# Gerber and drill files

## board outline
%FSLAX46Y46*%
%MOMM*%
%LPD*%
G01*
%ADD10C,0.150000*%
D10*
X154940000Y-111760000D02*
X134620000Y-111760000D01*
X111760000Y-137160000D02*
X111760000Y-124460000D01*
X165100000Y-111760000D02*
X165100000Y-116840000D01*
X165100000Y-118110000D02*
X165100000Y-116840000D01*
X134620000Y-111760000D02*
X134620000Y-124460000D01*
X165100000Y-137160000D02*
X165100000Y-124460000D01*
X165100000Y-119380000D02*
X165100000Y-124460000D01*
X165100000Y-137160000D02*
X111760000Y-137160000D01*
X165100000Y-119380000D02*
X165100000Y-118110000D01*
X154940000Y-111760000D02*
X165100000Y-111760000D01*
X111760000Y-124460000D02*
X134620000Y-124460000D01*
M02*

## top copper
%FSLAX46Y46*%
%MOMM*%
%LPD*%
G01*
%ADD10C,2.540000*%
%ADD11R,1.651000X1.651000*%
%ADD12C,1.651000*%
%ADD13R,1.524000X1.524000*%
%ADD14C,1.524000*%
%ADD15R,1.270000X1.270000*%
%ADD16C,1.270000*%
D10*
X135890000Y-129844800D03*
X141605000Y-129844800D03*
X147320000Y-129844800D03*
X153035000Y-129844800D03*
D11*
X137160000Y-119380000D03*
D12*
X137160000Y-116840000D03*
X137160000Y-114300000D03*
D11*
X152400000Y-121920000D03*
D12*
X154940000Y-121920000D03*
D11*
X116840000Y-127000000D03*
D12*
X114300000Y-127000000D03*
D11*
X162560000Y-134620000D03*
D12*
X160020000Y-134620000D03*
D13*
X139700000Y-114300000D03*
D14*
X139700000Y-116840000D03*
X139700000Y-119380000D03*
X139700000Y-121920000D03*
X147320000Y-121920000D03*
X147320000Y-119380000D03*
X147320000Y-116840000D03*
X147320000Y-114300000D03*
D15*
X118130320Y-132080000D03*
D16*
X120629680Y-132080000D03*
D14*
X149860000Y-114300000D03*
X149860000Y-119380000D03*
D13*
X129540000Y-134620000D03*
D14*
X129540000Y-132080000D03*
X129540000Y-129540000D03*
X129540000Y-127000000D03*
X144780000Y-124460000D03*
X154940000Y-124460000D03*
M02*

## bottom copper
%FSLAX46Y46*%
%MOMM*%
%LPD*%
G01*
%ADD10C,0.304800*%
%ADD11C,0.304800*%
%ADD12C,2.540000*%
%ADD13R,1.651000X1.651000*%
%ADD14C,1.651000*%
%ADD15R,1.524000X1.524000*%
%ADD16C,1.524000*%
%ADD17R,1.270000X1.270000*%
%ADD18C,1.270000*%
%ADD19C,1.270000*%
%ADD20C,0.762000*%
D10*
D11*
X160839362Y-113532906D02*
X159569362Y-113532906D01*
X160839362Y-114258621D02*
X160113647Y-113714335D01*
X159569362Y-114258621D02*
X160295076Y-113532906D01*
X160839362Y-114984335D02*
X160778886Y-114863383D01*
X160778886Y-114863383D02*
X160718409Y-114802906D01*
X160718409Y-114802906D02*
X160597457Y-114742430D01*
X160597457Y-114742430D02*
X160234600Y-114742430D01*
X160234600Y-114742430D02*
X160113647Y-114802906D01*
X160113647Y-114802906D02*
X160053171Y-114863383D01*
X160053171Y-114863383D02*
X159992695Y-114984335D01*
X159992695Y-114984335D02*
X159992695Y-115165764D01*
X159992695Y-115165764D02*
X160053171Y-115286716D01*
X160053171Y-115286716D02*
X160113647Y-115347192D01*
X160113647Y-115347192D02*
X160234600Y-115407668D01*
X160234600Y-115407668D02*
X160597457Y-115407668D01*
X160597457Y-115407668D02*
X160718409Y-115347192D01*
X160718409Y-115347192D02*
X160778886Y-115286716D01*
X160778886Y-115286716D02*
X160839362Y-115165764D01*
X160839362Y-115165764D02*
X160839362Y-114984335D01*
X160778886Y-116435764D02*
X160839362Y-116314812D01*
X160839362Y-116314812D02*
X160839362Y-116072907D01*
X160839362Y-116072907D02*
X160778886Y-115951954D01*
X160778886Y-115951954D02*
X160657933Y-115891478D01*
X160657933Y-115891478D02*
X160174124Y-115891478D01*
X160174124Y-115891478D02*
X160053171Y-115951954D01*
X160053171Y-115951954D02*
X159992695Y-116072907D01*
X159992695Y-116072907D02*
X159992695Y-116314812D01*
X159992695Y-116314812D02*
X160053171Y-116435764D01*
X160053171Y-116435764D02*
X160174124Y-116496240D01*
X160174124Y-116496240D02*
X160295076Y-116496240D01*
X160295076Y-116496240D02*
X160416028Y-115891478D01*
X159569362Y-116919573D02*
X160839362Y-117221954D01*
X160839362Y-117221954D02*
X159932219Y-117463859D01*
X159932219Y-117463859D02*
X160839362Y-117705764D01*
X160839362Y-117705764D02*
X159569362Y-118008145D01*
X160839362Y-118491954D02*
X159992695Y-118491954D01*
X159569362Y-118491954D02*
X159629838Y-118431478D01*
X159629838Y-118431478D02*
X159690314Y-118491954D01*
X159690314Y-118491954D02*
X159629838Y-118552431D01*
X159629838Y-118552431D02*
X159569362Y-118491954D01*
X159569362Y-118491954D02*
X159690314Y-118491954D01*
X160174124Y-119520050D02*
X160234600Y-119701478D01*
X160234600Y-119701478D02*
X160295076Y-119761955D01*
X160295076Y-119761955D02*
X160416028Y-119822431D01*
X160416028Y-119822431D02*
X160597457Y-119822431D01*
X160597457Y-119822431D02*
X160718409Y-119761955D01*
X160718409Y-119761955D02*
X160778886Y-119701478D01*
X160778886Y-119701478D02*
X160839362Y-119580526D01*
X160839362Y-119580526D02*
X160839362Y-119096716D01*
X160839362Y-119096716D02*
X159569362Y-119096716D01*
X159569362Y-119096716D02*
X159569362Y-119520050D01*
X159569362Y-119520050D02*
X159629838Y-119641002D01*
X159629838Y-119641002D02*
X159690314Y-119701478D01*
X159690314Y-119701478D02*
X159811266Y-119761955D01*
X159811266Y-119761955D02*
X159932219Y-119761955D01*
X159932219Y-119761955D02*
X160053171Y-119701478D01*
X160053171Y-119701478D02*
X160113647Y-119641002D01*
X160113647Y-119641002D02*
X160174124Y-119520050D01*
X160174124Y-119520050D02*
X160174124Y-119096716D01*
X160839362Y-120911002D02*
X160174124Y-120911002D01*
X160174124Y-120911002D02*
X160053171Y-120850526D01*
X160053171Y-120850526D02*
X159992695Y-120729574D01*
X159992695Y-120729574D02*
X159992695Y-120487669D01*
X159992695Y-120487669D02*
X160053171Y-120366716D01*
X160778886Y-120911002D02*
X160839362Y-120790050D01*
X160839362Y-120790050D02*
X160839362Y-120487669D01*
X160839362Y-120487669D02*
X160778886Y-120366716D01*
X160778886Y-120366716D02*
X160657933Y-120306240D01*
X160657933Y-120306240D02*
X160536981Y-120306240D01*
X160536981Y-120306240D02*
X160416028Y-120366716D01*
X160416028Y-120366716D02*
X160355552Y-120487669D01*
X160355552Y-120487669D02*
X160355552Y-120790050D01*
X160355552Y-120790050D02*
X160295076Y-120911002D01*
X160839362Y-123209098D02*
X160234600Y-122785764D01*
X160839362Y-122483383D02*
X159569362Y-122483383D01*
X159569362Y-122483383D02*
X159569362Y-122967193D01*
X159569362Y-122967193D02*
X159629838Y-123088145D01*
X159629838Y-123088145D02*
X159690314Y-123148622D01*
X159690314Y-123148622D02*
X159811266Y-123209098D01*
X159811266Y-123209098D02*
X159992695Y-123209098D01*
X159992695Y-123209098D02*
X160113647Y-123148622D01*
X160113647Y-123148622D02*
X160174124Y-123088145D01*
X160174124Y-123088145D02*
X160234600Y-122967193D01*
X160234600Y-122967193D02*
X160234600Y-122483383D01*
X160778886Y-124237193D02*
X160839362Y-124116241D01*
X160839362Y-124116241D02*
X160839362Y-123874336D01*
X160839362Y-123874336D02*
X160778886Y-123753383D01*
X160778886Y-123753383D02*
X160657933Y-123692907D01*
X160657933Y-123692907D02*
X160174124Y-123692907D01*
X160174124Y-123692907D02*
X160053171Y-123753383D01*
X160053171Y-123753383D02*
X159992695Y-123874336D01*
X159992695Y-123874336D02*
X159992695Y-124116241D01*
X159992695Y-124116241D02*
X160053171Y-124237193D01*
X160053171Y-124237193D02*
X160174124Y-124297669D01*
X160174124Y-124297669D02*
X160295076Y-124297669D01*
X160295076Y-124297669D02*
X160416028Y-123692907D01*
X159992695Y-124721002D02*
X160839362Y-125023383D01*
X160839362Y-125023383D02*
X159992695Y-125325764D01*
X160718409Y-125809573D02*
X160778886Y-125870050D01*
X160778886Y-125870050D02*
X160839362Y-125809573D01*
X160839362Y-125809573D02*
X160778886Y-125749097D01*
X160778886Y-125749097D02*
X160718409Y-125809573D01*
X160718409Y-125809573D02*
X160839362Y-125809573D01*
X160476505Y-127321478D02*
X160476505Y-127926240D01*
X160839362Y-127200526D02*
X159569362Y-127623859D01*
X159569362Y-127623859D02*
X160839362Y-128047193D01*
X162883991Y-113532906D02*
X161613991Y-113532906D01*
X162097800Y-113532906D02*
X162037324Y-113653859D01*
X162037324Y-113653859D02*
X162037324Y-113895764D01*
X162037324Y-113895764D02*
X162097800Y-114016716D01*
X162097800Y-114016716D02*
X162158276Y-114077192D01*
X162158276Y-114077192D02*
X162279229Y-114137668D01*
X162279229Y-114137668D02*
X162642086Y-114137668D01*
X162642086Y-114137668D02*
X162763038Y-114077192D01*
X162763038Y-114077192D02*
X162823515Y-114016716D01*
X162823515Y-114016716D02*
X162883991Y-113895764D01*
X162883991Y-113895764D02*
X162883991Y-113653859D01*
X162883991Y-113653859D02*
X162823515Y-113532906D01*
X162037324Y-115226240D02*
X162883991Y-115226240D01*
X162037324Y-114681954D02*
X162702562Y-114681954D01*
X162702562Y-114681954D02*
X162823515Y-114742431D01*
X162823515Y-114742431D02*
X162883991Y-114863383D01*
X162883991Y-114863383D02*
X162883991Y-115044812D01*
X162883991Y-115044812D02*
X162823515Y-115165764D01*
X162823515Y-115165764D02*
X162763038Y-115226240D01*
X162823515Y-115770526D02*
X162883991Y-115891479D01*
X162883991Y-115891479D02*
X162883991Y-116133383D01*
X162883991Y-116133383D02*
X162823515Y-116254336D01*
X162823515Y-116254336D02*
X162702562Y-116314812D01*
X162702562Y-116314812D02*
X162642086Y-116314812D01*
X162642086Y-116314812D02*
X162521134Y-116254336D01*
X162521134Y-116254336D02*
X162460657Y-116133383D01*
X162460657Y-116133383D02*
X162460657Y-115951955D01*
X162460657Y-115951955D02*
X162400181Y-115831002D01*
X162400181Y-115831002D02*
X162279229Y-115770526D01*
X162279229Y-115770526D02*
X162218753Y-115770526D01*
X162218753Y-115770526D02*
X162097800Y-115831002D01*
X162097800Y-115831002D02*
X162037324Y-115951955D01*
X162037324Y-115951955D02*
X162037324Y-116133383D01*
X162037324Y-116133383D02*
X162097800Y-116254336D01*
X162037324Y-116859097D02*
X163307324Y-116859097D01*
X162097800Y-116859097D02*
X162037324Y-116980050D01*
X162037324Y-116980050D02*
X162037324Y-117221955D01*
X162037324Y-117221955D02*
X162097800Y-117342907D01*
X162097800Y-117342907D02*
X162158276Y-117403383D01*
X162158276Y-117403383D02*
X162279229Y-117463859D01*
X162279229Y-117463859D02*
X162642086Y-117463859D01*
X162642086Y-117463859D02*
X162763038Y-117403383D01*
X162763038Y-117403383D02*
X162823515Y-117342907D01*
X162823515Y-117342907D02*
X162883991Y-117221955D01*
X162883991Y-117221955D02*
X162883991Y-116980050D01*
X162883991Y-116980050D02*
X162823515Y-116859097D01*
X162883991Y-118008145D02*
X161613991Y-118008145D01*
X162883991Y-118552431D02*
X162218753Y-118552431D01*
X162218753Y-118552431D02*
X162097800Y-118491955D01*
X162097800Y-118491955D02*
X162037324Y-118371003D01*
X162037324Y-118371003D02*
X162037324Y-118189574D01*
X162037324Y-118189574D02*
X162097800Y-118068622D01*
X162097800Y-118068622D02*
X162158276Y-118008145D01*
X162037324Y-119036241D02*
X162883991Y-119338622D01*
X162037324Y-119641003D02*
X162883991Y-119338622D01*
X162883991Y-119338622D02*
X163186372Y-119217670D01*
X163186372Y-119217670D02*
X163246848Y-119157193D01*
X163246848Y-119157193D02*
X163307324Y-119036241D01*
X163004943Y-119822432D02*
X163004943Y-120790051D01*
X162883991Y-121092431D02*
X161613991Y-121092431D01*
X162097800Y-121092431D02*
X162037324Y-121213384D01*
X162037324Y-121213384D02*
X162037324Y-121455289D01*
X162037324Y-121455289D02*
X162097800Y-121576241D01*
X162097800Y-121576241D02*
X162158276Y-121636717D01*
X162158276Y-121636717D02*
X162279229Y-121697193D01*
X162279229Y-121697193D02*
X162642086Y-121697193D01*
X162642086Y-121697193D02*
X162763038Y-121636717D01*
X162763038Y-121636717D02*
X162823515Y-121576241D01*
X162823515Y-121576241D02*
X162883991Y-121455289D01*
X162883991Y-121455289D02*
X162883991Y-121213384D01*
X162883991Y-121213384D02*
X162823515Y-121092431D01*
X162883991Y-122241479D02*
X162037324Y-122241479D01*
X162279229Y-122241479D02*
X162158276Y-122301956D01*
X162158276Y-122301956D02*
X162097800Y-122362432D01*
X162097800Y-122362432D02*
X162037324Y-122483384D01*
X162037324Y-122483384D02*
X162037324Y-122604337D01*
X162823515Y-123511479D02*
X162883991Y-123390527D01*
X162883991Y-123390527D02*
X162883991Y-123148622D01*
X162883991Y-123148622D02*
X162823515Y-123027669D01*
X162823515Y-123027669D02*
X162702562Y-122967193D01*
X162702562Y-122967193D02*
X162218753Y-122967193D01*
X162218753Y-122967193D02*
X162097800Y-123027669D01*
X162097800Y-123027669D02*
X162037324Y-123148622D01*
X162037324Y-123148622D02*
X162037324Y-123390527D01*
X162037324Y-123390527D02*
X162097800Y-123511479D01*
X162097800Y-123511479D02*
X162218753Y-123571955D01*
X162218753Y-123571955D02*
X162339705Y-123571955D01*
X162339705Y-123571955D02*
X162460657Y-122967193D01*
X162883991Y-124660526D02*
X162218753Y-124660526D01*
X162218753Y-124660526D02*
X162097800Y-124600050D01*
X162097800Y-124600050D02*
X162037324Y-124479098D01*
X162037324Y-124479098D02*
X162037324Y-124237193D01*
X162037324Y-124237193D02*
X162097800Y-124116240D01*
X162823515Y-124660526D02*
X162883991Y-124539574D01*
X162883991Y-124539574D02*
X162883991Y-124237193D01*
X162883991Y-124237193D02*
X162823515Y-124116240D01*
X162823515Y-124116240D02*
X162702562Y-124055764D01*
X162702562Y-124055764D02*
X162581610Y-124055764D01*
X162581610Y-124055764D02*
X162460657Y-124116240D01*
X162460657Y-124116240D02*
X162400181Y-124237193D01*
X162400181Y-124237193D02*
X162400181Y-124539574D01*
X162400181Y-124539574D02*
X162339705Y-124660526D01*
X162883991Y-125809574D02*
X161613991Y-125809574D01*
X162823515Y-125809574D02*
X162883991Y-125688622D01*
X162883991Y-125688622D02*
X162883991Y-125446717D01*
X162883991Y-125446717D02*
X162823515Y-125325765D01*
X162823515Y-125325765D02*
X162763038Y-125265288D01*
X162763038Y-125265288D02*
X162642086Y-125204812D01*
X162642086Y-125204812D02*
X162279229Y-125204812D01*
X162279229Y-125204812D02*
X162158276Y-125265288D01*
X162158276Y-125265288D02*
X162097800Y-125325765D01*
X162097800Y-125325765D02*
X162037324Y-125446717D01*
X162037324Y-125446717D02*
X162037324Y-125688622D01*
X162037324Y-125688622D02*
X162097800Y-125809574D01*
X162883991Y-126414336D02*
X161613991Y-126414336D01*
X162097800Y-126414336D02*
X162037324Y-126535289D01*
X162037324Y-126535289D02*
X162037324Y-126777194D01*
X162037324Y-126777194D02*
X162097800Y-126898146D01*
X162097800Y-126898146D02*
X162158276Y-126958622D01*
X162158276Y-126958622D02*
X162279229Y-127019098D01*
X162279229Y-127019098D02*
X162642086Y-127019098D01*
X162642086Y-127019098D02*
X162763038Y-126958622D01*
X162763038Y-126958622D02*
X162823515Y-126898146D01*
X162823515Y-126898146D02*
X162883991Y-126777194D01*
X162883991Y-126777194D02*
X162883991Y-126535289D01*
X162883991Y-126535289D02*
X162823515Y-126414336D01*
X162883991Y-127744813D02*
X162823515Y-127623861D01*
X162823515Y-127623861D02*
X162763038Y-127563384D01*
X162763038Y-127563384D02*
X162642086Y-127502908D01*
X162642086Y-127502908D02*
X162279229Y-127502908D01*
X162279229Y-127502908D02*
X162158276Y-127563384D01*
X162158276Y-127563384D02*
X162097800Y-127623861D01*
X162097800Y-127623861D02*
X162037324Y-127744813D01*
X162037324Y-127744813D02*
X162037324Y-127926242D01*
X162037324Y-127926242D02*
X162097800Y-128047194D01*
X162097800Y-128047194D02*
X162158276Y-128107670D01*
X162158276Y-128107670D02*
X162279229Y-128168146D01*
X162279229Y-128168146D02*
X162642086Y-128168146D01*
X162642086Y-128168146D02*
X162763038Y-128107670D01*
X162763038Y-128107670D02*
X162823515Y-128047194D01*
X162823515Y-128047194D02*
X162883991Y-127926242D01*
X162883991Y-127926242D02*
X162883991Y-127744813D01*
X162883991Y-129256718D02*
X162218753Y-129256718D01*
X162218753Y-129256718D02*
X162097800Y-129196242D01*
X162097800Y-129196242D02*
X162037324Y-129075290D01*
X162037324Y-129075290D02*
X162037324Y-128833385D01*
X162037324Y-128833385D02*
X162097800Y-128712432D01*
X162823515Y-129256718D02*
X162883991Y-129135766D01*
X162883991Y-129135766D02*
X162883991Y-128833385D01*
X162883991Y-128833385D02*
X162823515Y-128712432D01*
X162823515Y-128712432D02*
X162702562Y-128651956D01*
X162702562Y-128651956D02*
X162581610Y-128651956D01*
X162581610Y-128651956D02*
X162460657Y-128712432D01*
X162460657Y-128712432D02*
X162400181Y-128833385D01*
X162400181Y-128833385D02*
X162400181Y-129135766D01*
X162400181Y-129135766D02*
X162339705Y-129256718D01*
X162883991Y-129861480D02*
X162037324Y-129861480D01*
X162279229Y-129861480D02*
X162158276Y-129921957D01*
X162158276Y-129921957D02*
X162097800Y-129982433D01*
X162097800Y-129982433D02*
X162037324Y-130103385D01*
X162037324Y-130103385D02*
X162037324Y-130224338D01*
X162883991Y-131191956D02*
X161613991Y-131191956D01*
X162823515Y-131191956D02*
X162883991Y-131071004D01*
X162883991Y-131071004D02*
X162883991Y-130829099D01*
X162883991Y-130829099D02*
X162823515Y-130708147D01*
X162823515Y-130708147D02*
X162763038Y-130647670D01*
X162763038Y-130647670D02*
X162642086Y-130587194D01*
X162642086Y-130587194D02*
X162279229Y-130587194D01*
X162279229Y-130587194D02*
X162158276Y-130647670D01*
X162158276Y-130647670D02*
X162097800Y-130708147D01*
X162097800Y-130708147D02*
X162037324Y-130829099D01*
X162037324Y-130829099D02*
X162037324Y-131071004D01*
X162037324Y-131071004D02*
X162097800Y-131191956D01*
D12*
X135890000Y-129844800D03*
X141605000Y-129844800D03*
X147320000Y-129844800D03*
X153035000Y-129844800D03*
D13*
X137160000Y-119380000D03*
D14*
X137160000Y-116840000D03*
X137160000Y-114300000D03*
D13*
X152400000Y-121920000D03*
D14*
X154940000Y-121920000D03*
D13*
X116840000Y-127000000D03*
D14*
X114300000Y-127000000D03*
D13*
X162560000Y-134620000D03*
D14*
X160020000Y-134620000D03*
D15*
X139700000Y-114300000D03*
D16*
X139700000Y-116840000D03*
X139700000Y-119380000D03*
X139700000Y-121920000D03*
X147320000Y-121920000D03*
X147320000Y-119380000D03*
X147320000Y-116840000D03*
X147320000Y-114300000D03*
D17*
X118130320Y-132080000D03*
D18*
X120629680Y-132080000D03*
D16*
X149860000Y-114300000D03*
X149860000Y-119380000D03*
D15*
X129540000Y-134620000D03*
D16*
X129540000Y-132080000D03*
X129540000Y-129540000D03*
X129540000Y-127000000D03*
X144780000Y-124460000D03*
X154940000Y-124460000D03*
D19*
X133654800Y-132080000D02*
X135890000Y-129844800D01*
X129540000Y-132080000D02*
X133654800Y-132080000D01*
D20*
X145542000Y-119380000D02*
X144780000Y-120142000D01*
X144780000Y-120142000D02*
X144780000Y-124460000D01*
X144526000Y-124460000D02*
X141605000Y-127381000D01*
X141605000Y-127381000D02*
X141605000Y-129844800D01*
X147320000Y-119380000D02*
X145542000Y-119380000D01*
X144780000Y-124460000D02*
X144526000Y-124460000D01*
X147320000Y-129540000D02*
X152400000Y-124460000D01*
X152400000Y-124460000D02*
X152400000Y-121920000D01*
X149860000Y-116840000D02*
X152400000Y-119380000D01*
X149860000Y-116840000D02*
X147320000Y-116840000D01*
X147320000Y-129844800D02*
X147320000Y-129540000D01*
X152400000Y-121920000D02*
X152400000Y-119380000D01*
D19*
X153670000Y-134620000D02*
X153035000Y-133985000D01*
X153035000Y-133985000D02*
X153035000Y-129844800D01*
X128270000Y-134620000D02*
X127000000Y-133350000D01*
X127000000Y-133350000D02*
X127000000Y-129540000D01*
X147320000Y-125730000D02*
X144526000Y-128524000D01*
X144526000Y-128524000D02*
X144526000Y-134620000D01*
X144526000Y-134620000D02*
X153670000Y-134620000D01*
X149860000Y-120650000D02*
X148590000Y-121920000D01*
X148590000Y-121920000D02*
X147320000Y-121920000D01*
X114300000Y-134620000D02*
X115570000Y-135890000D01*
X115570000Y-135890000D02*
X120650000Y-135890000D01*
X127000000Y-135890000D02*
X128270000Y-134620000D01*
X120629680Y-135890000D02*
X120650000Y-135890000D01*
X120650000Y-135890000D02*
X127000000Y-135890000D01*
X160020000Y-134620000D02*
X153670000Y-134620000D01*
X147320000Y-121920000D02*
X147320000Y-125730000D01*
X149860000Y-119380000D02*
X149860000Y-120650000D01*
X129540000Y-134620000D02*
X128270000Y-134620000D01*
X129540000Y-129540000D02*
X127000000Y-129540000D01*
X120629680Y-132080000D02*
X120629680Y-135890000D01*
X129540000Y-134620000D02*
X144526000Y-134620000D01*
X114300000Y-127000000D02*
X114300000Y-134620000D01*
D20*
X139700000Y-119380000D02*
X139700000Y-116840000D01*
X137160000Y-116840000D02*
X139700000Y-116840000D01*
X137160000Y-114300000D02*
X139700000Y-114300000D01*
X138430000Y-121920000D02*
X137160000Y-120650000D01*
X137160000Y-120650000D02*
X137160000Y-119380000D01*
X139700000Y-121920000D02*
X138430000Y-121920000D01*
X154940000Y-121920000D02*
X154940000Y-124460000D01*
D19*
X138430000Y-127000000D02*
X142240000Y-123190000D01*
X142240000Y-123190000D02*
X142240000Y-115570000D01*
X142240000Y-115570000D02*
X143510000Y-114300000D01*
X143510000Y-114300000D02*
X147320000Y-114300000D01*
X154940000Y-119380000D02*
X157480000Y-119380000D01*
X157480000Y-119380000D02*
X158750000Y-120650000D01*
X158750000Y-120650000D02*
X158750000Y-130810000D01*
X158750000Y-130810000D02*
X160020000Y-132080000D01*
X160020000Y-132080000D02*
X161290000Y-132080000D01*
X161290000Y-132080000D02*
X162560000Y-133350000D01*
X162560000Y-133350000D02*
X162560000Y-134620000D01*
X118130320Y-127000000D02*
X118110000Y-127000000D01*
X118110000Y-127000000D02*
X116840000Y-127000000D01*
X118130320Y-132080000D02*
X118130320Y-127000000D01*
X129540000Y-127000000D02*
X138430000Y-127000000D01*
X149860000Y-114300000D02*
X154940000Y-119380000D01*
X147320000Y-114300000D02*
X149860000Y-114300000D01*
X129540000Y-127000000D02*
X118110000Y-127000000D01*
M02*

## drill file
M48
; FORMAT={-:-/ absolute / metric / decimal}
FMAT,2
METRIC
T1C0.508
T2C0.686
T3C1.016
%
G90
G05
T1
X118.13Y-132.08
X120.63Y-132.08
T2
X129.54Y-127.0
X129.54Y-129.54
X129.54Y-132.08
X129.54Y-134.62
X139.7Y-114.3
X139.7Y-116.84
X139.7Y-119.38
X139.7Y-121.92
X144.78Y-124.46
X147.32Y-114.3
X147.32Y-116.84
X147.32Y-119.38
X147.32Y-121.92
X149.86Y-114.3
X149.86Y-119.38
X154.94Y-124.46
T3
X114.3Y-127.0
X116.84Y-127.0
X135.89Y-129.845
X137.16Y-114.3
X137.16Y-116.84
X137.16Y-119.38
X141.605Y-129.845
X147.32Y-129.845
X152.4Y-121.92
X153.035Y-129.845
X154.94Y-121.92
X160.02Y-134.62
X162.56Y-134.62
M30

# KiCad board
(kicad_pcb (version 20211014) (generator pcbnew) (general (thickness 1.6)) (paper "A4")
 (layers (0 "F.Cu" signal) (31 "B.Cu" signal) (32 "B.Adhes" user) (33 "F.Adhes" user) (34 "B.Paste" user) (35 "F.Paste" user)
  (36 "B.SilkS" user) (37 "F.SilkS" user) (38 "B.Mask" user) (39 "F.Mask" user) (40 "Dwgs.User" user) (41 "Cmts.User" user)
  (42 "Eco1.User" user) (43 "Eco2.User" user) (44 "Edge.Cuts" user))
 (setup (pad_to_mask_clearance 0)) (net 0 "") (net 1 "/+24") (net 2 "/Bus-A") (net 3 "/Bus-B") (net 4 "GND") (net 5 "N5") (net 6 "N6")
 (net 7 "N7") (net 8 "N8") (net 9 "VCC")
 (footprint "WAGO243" (layer "F.Cu") (at 133.35 126.365)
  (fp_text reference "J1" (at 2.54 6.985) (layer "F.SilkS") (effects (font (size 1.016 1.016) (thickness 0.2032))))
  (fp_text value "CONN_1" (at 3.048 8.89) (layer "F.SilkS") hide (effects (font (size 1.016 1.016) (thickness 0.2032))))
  (pad "1" thru_hole circle locked (at 2.54 3.4798) (size 2.54 2.54) (drill 1.016) (layers *.Cu *.Mask "F.SilkS") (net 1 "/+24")))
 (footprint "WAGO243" (layer "F.Cu") (at 139.065 126.365)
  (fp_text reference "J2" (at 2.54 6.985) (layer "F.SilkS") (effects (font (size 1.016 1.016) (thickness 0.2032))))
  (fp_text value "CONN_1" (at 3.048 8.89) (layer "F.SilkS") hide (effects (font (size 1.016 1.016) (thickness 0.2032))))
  (pad "1" thru_hole circle locked (at 2.54 3.4798) (size 2.54 2.54) (drill 1.016) (layers *.Cu *.Mask "F.SilkS") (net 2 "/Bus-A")))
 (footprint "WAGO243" (layer "F.Cu") (at 144.78 126.365)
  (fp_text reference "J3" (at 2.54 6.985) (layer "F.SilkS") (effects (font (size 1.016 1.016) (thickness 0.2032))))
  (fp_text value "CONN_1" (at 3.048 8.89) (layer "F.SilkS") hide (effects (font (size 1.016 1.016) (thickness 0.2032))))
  (pad "1" thru_hole circle locked (at 2.54 3.4798) (size 2.54 2.54) (drill 1.016) (layers *.Cu *.Mask "F.SilkS") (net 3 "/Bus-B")))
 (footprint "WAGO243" (layer "F.Cu") (at 150.495 126.365)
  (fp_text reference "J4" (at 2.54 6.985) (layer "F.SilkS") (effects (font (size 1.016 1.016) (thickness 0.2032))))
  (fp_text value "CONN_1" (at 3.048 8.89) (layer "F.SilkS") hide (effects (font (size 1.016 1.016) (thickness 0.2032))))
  (pad "1" thru_hole circle locked (at 2.54 3.4798) (size 2.54 2.54) (drill 1.016) (layers *.Cu *.Mask "F.SilkS") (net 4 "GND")))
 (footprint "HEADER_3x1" (layer "F.Cu") (at 137.16 119.38 90)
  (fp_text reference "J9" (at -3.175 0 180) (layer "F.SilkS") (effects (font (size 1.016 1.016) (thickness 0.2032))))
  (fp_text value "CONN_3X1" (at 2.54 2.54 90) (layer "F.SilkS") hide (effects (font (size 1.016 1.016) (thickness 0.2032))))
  (pad "1" thru_hole rect locked (at 0 0 90) (size 1.651 1.651) (drill 1.016) (layers *.Cu *.Mask "F.SilkS") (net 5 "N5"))
  (pad "2" thru_hole circle locked (at 2.54 0 90) (size 1.651 1.651) (drill 1.016) (layers *.Cu *.Mask "F.SilkS") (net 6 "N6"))
  (pad "3" thru_hole circle locked (at 5.08 0 90) (size 1.651 1.651) (drill 1.016) (layers *.Cu *.Mask "F.SilkS") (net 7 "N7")))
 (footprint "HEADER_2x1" (layer "F.Cu") (at 152.4 121.92)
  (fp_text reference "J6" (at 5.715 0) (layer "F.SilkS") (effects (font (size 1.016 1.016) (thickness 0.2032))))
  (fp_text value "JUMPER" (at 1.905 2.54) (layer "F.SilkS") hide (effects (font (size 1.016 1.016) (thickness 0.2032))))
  (pad "1" thru_hole rect locked (at 0 0) (size 1.651 1.651) (drill 1.016) (layers *.Cu *.Mask "F.SilkS") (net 3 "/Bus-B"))
  (pad "2" thru_hole circle locked (at 2.54 0) (size 1.651 1.651) (drill 1.016) (layers *.Cu *.Mask "F.SilkS") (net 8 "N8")))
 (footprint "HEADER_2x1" (layer "F.Cu") (at 116.84 127 180)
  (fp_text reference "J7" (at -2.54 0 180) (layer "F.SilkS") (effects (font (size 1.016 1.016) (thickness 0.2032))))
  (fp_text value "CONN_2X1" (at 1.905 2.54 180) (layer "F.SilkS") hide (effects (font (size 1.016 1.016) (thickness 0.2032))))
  (pad "1" thru_hole rect locked (at 0 0 180) (size 1.651 1.651) (drill 1.016) (layers *.Cu *.Mask "F.SilkS") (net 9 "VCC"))
  (pad "2" thru_hole circle locked (at 2.54 0 180) (size 1.651 1.651) (drill 1.016) (layers *.Cu *.Mask "F.SilkS") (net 4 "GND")))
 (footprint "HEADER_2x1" (layer "F.Cu") (at 162.56 134.62 180)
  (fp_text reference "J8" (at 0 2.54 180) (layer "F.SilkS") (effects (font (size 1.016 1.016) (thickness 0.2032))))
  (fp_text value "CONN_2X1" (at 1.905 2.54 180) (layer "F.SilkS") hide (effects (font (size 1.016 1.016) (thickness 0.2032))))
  (pad "1" thru_hole rect locked (at 0 0 180) (size 1.651 1.651) (drill 1.016) (layers *.Cu *.Mask "F.SilkS") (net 9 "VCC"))
  (pad "2" thru_hole circle locked (at 2.54 0 180) (size 1.651 1.651) (drill 1.016) (layers *.Cu *.Mask "F.SilkS") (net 4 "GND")))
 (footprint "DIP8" (layer "F.Cu") (at 139.7 114.3 -90)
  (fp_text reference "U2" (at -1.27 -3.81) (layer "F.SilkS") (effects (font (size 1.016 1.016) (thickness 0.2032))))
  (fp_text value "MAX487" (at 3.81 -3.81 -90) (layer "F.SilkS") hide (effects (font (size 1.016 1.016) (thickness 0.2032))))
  (pad "1" thru_hole rect locked (at 0 0 270) (size 1.524 1.524) (drill 0.6858) (layers *.Cu *.Mask "F.SilkS") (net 7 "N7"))
  (pad "2" thru_hole circle locked (at 2.54 0 270) (size 1.524 1.524) (drill 0.6858) (layers *.Cu *.Mask "F.SilkS") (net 6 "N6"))
  (pad "3" thru_hole circle locked (at 5.08 0 270) (size 1.524 1.524) (drill 0.6858) (layers *.Cu *.Mask "F.SilkS") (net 6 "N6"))
  (pad "4" thru_hole circle locked (at 7.62 0 270) (size 1.524 1.524) (drill 0.6858) (layers *.Cu *.Mask "F.SilkS") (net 5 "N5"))
  (pad "5" thru_hole circle locked (at 7.62 -7.62 270) (size 1.524 1.524) (drill 0.6858) (layers *.Cu *.Mask "F.SilkS") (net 4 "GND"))
  (pad "6" thru_hole circle locked (at 5.08 -7.62 270) (size 1.524 1.524) (drill 0.6858) (layers *.Cu *.Mask "F.SilkS") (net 2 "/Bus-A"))
  (pad "7" thru_hole circle locked (at 2.54 -7.62 270) (size 1.524 1.524) (drill 0.6858) (layers *.Cu *.Mask "F.SilkS") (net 3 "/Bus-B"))
  (pad "8" thru_hole circle locked (at 0 -7.62 270) (size 1.524 1.524) (drill 0.6858) (layers *.Cu *.Mask "F.SilkS") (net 9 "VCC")))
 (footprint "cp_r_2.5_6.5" (layer "F.Cu") (at 119.38 132.08)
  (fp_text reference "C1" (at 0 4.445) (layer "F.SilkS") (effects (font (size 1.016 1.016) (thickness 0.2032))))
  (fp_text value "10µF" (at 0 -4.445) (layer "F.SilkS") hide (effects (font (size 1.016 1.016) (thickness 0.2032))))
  (pad "1" thru_hole rect locked (at -1.24968 0) (size 1.27 1.27) (drill 0.508) (layers *.Cu *.Mask "F.SilkS") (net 9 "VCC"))
  (pad "2" thru_hole circle locked (at 1.24968 0) (size 1.27 1.27) (drill 0.508) (layers *.Cu *.Mask "F.SilkS") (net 4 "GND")))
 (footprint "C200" (layer "F.Cu") (at 149.86 114.3 -90)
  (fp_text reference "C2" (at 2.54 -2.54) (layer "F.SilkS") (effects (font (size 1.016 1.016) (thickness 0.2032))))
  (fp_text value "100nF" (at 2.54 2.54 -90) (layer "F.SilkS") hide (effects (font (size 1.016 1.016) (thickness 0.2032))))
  (pad "1" thru_hole circle locked (at 0 0 270) (size 1.524 1.524) (drill 0.6858) (layers *.Cu *.Mask "F.SilkS") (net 9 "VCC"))
  (pad "2" thru_hole circle locked (at 5.08 0 270) (size 1.524 1.524) (drill 0.6858) (layers *.Cu *.Mask "F.SilkS") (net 4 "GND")))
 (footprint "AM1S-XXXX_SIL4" (layer "F.Cu") (at 129.54 134.62 90)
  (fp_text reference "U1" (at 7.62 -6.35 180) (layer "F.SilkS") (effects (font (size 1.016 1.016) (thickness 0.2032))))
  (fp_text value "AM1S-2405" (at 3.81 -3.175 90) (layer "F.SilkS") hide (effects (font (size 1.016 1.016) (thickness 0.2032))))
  (pad "1" thru_hole rect locked (at 0 0 90) (size 1.524 1.524) (drill 0.6858) (layers *.Cu *.Mask "F.SilkS") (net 4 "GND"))
  (pad "2" thru_hole circle locked (at 2.54 0 90) (size 1.524 1.524) (drill 0.6858) (layers *.Cu *.Mask "F.SilkS") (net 1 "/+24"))
  (pad "3" thru_hole circle locked (at 5.08 0 90) (size 1.524 1.524) (drill 0.6858) (layers *.Cu *.Mask "F.SilkS") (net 4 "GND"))
  (pad "4" thru_hole circle locked (at 7.62 0 90) (size 1.524 1.524) (drill 0.6858) (layers *.Cu *.Mask "F.SilkS") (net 9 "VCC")))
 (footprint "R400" (layer "F.Cu") (at 144.78 124.46)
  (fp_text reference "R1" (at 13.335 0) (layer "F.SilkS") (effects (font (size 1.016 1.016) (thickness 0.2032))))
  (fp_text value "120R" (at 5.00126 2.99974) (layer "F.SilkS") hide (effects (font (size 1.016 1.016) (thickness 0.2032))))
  (pad "1" thru_hole circle locked (at 0 0) (size 1.524 1.524) (drill 0.6858) (layers *.Cu *.Mask "F.SilkS") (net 2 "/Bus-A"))
  (pad "2" thru_hole circle locked (at 10.16 0) (size 1.524 1.524) (drill 0.6858) (layers *.Cu *.Mask "F.SilkS") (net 8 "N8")))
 (gr_line (start 154.94 111.76) (end 134.62 111.76) (layer "Edge.Cuts") (width 0.15))
 (gr_line (start 111.76 137.16) (end 111.76 124.46) (layer "Edge.Cuts") (width 0.15))
 (gr_line (start 165.1 111.76) (end 165.1 116.84) (layer "Edge.Cuts") (width 0.15))
 (gr_line (start 165.1 118.11) (end 165.1 116.84) (layer "Edge.Cuts") (width 0.15))
 (gr_line (start 134.62 111.76) (end 134.62 124.46) (layer "Edge.Cuts") (width 0.15))
 (gr_line (start 165.1 137.16) (end 165.1 124.46) (layer "Edge.Cuts") (width 0.15))
 (gr_line (start 165.1 119.38) (end 165.1 124.46) (layer "Edge.Cuts") (width 0.15))
 (gr_line (start 165.1 137.16) (end 111.76 137.16) (layer "Edge.Cuts") (width 0.15))
 (gr_line (start 165.1 119.38) (end 165.1 118.11) (layer "Edge.Cuts") (width 0.15))
 (gr_line (start 154.94 111.76) (end 165.1 111.76) (layer "Edge.Cuts") (width 0.15))
 (gr_line (start 111.76 124.46) (end 134.62 124.46) (layer "Edge.Cuts") (width 0.15))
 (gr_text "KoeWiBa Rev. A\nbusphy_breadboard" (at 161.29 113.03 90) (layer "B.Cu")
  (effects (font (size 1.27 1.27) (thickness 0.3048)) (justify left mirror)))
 (segment (start 133.6548 132.08) (end 135.89 129.8448) (width 1.27) (layer "B.Cu") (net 1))
 (segment (start 129.54 132.08) (end 133.6548 132.08) (width 1.27) (layer "B.Cu") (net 1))
 (segment (start 145.542 119.38) (end 144.78 120.142) (width 0.762) (layer "B.Cu") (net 2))
 (segment (start 144.78 120.142) (end 144.78 124.46) (width 0.762) (layer "B.Cu") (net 2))
 (segment (start 144.526 124.46) (end 141.605 127.381) (width 0.762) (layer "B.Cu") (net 2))
 (segment (start 141.605 127.381) (end 141.605 129.8448) (width 0.762) (layer "B.Cu") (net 2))
 (segment (start 147.32 119.38) (end 145.542 119.38) (width 0.762) (layer "B.Cu") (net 2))
 (segment (start 144.78 124.46) (end 144.526 124.46) (width 0.762) (layer "B.Cu") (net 2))
 (segment (start 147.32 129.54) (end 152.4 124.46) (width 0.762) (layer "B.Cu") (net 3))
 (segment (start 152.4 124.46) (end 152.4 121.92) (width 0.762) (layer "B.Cu") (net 3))
 (segment (start 149.86 116.84) (end 152.4 119.38) (width 0.762) (layer "B.Cu") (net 3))
 (segment (start 149.86 116.84) (end 147.32 116.84) (width 0.762) (layer "B.Cu") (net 3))
 (segment (start 147.32 129.8448) (end 147.32 129.54) (width 0.762) (layer "B.Cu") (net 3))
 (segment (start 152.4 121.92) (end 152.4 119.38) (width 0.762) (layer "B.Cu") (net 3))
 (segment (start 153.67 134.62) (end 153.035 133.985) (width 1.27) (layer "B.Cu") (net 4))
 (segment (start 153.035 133.985) (end 153.035 129.8448) (width 1.27) (layer "B.Cu") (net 4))
 (segment (start 128.27 134.62) (end 127 133.35) (width 1.27) (layer "B.Cu") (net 4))
 (segment (start 127 133.35) (end 127 129.54) (width 1.27) (layer "B.Cu") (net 4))
 (segment (start 147.32 125.73) (end 144.526 128.524) (width 1.27) (layer "B.Cu") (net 4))
 (segment (start 144.526 128.524) (end 144.526 134.62) (width 1.27) (layer "B.Cu") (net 4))
 (segment (start 144.526 134.62) (end 153.67 134.62) (width 1.27) (layer "B.Cu") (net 4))
 (segment (start 149.86 120.65) (end 148.59 121.92) (width 1.27) (layer "B.Cu") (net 4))
 (segment (start 148.59 121.92) (end 147.32 121.92) (width 1.27) (layer "B.Cu") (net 4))
 (segment (start 114.3 134.62) (end 115.57 135.89) (width 1.27) (layer "B.Cu") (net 4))
 (segment (start 115.57 135.89) (end 120.65 135.89) (width 1.27) (layer "B.Cu") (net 4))
 (segment (start 127 135.89) (end 128.27 134.62) (width 1.27) (layer "B.Cu") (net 4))
 (segment (start 120.62968 135.89) (end 120.65 135.89) (width 1.27) (layer "B.Cu") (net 4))
 (segment (start 120.65 135.89) (end 127 135.89) (width 1.27) (layer "B.Cu") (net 4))
 (segment (start 160.02 134.62) (end 153.67 134.62) (width 1.27) (layer "B.Cu") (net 4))
 (segment (start 147.32 121.92) (end 147.32 125.73) (width 1.27) (layer "B.Cu") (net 4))
 (segment (start 149.86 119.38) (end 149.86 120.65) (width 1.27) (layer "B.Cu") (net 4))
 (segment (start 129.54 134.62) (end 128.27 134.62) (width 1.27) (layer "B.Cu") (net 4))
 (segment (start 129.54 129.54) (end 127 129.54) (width 1.27) (layer "B.Cu") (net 4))
 (segment (start 120.62968 132.08) (end 120.62968 135.89) (width 1.27) (layer "B.Cu") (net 4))
 (segment (start 129.54 134.62) (end 144.526 134.62) (width 1.27) (layer "B.Cu") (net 4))
 (segment (start 114.3 127) (end 114.3 134.62) (width 1.27) (layer "B.Cu") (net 4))
 (segment (start 139.7 119.38) (end 139.7 116.84) (width 0.762) (layer "B.Cu") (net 6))
 (segment (start 137.16 116.84) (end 139.7 116.84) (width 0.762) (layer "B.Cu") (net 6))
 (segment (start 137.16 114.3) (end 139.7 114.3) (width 0.762) (layer "B.Cu") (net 7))
 (segment (start 138.43 121.92) (end 137.16 120.65) (width 0.762) (layer "B.Cu") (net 5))
 (segment (start 137.16 120.65) (end 137.16 119.38) (width 0.762) (layer "B.Cu") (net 5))
 (segment (start 139.7 121.92) (end 138.43 121.92) (width 0.762) (layer "B.Cu") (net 5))
 (segment (start 154.94 121.92) (end 154.94 124.46) (width 0.762) (layer "B.Cu") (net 8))
 (segment (start 138.43 127) (end 142.24 123.19) (width 1.27) (layer "B.Cu") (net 9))
 (segment (start 142.24 123.19) (end 142.24 115.57) (width 1.27) (layer "B.Cu") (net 9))
 (segment (start 142.24 115.57) (end 143.51 114.3) (width 1.27) (layer "B.Cu") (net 9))
 (segment (start 143.51 114.3) (end 147.32 114.3) (width 1.27) (layer "B.Cu") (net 9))
 (segment (start 154.94 119.38) (end 157.48 119.38) (width 1.27) (layer "B.Cu") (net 9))
 (segment (start 157.48 119.38) (end 158.75 120.65) (width 1.27) (layer "B.Cu") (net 9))
 (segment (start 158.75 120.65) (end 158.75 130.81) (width 1.27) (layer "B.Cu") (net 9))
 (segment (start 158.75 130.81) (end 160.02 132.08) (width 1.27) (layer "B.Cu") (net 9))
 (segment (start 160.02 132.08) (end 161.29 132.08) (width 1.27) (layer "B.Cu") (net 9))
 (segment (start 161.29 132.08) (end 162.56 133.35) (width 1.27) (layer "B.Cu") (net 9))
 (segment (start 162.56 133.35) (end 162.56 134.62) (width 1.27) (layer "B.Cu") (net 9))
 (segment (start 118.13032 127) (end 118.11 127) (width 1.27) (layer "B.Cu") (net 9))
 (segment (start 118.11 127) (end 116.84 127) (width 1.27) (layer "B.Cu") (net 9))
 (segment (start 118.13032 132.08) (end 118.13032 127) (width 1.27) (layer "B.Cu") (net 9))
 (segment (start 129.54 127) (end 138.43 127) (width 1.27) (layer "B.Cu") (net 9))
 (segment (start 149.86 114.3) (end 154.94 119.38) (width 1.27) (layer "B.Cu") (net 9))
 (segment (start 147.32 114.3) (end 149.86 114.3) (width 1.27) (layer "B.Cu") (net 9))
 (segment (start 129.54 127) (end 118.11 127) (width 1.27) (layer "B.Cu") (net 9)))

